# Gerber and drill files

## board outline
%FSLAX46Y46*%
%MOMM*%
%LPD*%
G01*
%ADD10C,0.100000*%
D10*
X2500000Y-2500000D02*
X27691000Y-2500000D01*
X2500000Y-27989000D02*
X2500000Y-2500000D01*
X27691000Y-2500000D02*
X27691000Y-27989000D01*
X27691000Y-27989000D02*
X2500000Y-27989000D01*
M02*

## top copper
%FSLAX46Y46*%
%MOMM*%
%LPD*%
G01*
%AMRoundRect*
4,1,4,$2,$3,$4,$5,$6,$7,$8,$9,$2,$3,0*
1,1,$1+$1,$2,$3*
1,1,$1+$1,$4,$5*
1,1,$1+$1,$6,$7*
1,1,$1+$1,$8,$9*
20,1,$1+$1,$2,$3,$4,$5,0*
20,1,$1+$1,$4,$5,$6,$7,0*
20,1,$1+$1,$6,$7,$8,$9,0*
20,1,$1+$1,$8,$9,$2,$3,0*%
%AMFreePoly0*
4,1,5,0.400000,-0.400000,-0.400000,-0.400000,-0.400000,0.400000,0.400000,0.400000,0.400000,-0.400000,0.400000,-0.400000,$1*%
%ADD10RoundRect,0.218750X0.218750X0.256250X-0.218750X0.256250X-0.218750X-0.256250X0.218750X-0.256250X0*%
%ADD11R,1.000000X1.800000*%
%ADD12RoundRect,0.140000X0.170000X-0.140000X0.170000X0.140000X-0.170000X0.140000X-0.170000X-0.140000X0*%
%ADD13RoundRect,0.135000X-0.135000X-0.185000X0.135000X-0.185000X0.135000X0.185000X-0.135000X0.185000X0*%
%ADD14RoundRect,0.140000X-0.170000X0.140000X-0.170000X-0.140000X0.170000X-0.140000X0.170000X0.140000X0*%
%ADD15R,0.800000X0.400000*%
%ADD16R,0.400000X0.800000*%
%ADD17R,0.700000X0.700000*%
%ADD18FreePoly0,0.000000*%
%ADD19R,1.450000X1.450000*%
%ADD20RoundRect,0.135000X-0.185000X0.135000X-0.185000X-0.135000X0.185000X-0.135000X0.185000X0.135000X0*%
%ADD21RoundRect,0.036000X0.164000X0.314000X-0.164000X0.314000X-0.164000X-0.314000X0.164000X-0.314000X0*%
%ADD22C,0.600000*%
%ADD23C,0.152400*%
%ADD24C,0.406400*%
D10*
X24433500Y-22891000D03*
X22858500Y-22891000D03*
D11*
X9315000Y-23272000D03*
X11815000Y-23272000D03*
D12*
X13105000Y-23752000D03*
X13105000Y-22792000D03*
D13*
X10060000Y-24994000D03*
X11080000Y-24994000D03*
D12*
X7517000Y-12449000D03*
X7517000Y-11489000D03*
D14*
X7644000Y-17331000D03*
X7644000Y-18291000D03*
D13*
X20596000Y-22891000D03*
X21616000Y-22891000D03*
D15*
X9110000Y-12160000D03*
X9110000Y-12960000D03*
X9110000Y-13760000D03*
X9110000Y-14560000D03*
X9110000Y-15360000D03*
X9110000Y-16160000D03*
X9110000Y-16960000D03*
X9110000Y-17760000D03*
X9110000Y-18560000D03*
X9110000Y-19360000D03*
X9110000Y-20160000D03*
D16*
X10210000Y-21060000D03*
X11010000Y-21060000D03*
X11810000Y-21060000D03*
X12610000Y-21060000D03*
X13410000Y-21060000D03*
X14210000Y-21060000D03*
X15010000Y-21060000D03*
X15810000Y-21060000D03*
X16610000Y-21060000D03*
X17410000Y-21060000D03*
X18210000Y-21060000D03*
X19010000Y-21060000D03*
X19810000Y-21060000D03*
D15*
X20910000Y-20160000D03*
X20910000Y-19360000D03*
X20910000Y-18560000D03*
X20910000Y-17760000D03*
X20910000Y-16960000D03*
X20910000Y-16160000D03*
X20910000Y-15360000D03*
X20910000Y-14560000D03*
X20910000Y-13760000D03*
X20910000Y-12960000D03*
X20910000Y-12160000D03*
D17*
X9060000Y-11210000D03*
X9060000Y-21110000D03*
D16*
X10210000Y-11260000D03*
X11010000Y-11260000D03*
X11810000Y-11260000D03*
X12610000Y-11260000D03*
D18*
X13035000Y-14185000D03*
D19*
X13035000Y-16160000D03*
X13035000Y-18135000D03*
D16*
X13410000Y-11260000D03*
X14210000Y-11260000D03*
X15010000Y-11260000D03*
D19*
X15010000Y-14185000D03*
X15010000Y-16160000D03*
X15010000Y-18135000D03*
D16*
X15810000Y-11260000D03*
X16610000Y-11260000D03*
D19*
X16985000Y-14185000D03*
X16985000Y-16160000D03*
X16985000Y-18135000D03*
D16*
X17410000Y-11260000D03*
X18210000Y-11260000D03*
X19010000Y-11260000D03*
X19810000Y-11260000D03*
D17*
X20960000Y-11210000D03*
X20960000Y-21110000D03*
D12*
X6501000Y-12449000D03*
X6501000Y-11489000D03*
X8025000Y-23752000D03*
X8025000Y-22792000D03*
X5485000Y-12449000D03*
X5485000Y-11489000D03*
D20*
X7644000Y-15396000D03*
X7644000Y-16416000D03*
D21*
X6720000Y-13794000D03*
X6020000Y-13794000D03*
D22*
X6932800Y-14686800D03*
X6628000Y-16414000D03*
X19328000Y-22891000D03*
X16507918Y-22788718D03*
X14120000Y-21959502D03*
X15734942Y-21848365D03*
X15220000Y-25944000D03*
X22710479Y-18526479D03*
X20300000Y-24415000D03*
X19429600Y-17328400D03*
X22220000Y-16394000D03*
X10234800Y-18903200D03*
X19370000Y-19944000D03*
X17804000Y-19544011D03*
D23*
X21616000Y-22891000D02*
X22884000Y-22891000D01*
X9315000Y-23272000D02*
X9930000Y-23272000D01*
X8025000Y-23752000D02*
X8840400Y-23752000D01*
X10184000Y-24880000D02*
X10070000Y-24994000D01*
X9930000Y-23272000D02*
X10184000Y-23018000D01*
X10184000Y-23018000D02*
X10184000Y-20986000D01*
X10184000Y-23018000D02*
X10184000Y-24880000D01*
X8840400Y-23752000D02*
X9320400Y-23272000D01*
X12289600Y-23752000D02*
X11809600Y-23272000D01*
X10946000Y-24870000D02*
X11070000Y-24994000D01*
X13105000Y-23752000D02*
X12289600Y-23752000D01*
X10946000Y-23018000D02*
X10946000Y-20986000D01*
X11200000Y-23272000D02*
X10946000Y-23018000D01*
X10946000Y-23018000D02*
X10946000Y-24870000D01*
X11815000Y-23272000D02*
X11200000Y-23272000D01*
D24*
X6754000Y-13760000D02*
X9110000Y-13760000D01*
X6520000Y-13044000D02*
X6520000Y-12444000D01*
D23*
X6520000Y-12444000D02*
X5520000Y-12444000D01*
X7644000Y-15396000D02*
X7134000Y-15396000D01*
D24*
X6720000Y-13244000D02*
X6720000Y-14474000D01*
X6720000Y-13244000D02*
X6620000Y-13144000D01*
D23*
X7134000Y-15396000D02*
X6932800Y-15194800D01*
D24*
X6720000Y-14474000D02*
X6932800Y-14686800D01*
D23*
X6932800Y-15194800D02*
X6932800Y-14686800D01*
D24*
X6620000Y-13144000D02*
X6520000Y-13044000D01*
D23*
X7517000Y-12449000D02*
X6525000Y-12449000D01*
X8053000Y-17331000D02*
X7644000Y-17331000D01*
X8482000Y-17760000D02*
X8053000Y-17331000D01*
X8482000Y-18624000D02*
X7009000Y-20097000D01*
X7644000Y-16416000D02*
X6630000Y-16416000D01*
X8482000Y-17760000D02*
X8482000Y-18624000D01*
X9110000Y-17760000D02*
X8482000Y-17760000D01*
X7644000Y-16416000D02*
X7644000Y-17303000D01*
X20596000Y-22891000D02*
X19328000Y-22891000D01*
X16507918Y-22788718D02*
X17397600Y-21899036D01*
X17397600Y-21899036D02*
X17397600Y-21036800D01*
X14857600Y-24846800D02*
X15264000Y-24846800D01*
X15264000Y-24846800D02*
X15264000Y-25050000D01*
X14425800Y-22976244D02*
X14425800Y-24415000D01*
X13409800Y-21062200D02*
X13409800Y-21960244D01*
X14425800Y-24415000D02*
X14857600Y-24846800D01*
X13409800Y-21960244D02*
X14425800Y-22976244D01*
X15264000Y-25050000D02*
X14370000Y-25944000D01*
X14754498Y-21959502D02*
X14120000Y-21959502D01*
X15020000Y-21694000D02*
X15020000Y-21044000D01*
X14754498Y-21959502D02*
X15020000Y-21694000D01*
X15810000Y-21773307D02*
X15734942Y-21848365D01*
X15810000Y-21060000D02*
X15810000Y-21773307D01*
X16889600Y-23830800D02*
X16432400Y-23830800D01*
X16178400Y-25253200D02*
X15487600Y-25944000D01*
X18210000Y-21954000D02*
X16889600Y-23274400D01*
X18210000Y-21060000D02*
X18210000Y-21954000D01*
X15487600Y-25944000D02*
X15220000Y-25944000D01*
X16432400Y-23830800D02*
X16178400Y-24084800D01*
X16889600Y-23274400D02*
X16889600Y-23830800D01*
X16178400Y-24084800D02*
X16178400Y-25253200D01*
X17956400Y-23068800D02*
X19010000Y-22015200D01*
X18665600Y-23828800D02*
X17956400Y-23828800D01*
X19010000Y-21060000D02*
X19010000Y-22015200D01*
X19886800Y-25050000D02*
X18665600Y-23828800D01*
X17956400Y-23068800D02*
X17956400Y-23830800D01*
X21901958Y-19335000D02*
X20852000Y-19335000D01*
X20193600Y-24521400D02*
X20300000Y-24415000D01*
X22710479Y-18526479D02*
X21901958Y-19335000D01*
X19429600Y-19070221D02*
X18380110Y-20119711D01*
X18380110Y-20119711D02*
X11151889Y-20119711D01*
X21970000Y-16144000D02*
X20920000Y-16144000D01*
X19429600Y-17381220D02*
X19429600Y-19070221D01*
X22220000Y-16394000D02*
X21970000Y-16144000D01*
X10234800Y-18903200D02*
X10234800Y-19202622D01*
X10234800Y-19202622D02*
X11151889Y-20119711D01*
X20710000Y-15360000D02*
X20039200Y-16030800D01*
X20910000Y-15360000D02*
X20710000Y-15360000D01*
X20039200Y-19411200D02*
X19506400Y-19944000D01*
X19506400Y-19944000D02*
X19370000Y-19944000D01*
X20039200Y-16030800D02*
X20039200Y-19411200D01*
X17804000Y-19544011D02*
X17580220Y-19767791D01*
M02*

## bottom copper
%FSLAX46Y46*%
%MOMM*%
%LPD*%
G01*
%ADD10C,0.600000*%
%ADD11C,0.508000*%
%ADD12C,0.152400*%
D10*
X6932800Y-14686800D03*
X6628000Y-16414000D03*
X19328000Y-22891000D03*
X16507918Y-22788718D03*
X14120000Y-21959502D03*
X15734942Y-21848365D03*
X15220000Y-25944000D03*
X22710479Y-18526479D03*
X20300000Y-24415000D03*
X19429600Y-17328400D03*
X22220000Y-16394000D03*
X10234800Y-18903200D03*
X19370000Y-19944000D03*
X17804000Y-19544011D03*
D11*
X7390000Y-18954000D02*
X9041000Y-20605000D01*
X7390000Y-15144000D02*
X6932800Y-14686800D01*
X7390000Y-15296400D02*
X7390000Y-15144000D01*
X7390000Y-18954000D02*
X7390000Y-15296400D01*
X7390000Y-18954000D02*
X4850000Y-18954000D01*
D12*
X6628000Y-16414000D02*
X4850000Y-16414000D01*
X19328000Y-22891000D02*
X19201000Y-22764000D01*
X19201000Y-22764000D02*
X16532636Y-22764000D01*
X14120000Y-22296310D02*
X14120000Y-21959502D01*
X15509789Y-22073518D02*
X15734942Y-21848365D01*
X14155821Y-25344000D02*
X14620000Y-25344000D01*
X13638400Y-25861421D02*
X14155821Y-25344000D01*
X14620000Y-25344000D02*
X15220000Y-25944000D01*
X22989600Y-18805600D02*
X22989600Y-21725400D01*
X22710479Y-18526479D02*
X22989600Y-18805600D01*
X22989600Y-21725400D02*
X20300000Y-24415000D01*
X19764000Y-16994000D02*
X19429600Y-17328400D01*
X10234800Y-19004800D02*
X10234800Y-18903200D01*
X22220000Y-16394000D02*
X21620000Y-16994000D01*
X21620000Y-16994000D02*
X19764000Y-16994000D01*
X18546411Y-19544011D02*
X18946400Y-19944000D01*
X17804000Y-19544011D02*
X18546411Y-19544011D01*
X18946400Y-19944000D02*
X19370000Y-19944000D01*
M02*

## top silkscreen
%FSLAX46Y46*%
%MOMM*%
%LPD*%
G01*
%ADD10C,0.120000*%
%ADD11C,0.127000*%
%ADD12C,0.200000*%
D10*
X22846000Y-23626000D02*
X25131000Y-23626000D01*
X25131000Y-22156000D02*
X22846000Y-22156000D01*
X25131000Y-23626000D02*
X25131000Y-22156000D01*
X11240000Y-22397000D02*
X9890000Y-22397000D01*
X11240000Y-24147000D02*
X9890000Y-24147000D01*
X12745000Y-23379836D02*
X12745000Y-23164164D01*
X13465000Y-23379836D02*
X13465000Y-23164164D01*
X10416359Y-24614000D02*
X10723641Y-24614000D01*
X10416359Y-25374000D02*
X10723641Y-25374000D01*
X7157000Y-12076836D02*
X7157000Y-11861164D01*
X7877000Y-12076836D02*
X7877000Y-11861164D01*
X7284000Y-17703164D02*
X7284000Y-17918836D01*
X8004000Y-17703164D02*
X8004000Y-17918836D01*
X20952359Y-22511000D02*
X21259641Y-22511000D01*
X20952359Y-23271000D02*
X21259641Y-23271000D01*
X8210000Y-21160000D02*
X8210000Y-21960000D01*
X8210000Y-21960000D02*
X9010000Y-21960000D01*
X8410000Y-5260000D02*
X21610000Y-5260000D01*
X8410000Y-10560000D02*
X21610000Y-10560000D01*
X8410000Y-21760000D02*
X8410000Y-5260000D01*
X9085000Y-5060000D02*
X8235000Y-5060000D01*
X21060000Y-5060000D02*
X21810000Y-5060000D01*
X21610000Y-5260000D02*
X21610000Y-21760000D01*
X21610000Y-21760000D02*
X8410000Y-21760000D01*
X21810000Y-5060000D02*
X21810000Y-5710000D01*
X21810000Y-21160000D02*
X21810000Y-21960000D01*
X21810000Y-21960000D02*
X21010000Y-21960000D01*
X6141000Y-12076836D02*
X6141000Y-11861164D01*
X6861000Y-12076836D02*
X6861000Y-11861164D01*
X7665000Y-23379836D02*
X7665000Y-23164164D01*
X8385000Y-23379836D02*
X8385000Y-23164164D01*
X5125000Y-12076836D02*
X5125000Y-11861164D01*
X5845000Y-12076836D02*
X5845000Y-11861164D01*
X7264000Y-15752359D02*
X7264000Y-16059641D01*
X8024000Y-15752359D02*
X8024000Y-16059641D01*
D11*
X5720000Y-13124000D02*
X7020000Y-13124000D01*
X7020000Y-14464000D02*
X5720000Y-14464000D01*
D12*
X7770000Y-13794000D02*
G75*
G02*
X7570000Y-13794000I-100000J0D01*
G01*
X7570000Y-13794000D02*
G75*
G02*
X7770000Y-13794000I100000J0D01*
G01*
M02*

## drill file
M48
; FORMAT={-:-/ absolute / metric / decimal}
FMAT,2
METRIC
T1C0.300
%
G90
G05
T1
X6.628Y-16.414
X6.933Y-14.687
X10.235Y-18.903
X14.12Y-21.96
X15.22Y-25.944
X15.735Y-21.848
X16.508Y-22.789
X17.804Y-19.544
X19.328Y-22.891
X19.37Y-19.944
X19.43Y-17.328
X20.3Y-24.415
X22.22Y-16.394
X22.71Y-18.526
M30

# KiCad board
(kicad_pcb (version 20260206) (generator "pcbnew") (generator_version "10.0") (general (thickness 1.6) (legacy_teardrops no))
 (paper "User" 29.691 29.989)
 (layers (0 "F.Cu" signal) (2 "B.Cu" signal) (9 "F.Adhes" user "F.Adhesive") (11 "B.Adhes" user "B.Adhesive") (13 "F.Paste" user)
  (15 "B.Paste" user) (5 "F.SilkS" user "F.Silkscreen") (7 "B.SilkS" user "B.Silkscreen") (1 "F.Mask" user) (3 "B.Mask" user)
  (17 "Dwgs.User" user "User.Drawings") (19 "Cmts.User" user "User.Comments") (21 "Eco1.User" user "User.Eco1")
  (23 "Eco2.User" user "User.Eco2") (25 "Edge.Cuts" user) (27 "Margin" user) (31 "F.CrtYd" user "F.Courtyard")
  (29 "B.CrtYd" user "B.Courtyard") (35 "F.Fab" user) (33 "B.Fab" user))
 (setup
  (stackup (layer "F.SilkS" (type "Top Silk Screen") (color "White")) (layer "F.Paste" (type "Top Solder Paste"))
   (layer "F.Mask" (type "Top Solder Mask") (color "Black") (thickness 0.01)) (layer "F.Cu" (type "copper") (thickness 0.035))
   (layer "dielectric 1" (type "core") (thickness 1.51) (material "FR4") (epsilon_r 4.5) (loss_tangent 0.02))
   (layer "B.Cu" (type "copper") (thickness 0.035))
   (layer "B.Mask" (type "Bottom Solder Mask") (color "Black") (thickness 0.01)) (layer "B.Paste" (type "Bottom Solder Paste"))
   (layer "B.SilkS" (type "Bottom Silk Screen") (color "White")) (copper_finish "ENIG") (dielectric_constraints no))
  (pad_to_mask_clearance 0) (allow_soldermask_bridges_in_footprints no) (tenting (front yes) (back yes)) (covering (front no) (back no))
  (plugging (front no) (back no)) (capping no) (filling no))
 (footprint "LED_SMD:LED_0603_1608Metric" (layer "F.Cu") (at 23.646 22.891 180)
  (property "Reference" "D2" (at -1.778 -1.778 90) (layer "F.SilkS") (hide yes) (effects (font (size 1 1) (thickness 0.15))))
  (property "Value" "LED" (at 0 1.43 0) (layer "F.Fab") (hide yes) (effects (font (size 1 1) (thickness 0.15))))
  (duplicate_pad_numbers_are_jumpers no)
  (fp_line (start 0.8 -0.735) (end -1.485 -0.735) (stroke (width 0.12) (type solid)) (layer "F.SilkS"))
  (fp_line (start -1.485 0.735) (end 0.8 0.735) (stroke (width 0.12) (type solid)) (layer "F.SilkS"))
  (fp_line (start -1.485 -0.735) (end -1.485 0.735) (stroke (width 0.12) (type solid)) (layer "F.SilkS"))
  (pad "1" smd roundrect (at -0.7875 0 180) (size 0.875 0.95) (layers "F.Cu" "F.Mask" "F.Paste") (roundrect_rratio 0.25) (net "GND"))
  (pad "2" smd roundrect (at 0.7875 0 180) (size 0.875 0.95) (layers "F.Cu" "F.Mask" "F.Paste") (roundrect_rratio 0.25)
   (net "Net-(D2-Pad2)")))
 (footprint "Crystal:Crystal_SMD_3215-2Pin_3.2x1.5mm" (layer "F.Cu") (at 10.565 23.272 180)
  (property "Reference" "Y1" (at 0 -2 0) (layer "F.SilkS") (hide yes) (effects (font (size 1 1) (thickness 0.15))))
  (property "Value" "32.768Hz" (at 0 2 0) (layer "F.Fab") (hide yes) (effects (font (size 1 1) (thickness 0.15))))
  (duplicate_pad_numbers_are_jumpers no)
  (fp_line (start -0.675 0.875) (end 0.675 0.875) (stroke (width 0.12) (type solid)) (layer "F.SilkS"))
  (fp_line (start -0.675 -0.875) (end 0.675 -0.875) (stroke (width 0.12) (type solid)) (layer "F.SilkS"))
  (pad "1" smd rect (at 1.25 0 180) (size 1 1.8) (layers "F.Cu" "F.Mask" "F.Paste") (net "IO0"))
  (pad "2" smd rect (at -1.25 0 180) (size 1 1.8) (layers "F.Cu" "F.Mask" "F.Paste") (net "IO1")))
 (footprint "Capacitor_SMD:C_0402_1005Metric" (layer "F.Cu") (at 13.105 23.272 90)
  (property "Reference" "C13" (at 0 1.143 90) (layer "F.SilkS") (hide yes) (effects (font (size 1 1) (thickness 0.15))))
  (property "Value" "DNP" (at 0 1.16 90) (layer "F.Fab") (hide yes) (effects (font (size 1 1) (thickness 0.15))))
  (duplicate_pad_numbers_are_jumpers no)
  (fp_line (start -0.107836 -0.36) (end 0.107836 -0.36) (stroke (width 0.12) (type solid)) (layer "F.SilkS"))
  (fp_line (start -0.107836 0.36) (end 0.107836 0.36) (stroke (width 0.12) (type solid)) (layer "F.SilkS"))
  (pad "1" smd roundrect (at -0.48 0 90) (size 0.56 0.62) (layers "F.Cu" "F.Mask" "F.Paste") (roundrect_rratio 0.25) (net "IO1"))
  (pad "2" smd roundrect (at 0.48 0 90) (size 0.56 0.62) (layers "F.Cu" "F.Mask" "F.Paste") (roundrect_rratio 0.25) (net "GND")))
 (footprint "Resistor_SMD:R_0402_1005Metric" (layer "F.Cu") (at 10.57 24.994)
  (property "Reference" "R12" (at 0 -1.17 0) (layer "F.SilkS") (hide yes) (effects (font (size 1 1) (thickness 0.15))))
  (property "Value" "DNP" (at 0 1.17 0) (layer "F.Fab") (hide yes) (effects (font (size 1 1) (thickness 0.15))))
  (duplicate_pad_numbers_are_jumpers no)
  (fp_line (start -0.153641 -0.38) (end 0.153641 -0.38) (stroke (width 0.12) (type solid)) (layer "F.SilkS"))
  (fp_line (start -0.153641 0.38) (end 0.153641 0.38) (stroke (width 0.12) (type solid)) (layer "F.SilkS"))
  (pad "1" smd roundrect (at -0.51 0) (size 0.54 0.64) (layers "F.Cu" "F.Mask" "F.Paste") (roundrect_rratio 0.25) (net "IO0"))
  (pad "2" smd roundrect (at 0.51 0) (size 0.54 0.64) (layers "F.Cu" "F.Mask" "F.Paste") (roundrect_rratio 0.25) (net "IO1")))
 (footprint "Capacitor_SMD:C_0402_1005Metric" (layer "F.Cu") (at 7.517 11.969 90)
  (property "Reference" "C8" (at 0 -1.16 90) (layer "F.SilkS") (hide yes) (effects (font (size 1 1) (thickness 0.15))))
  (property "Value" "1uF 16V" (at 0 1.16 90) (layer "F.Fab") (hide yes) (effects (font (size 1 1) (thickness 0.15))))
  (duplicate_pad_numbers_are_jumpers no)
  (fp_line (start -0.107836 -0.36) (end 0.107836 -0.36) (stroke (width 0.12) (type solid)) (layer "F.SilkS"))
  (fp_line (start -0.107836 0.36) (end 0.107836 0.36) (stroke (width 0.12) (type solid)) (layer "F.SilkS"))
  (pad "1" smd roundrect (at -0.48 0 90) (size 0.56 0.62) (layers "F.Cu" "F.Mask" "F.Paste") (roundrect_rratio 0.25) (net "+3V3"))
  (pad "2" smd roundrect (at 0.48 0 90) (size 0.56 0.62) (layers "F.Cu" "F.Mask" "F.Paste") (roundrect_rratio 0.25) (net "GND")))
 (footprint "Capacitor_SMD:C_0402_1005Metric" (layer "F.Cu") (at 7.644 17.811 -90)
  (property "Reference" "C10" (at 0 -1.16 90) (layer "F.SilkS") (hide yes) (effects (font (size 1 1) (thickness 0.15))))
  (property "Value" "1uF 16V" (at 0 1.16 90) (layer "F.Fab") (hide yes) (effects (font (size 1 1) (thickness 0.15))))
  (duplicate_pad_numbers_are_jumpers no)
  (fp_line (start -0.107836 0.36) (end 0.107836 0.36) (stroke (width 0.12) (type solid)) (layer "F.SilkS"))
  (fp_line (start -0.107836 -0.36) (end 0.107836 -0.36) (stroke (width 0.12) (type solid)) (layer "F.SilkS"))
  (pad "1" smd roundrect (at -0.48 0 270) (size 0.56 0.62) (layers "F.Cu" "F.Mask" "F.Paste") (roundrect_rratio 0.25) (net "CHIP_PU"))
  (pad "2" smd roundrect (at 0.48 0 270) (size 0.56 0.62) (layers "F.Cu" "F.Mask" "F.Paste") (roundrect_rratio 0.25) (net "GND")))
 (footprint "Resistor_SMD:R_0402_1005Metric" (layer "F.Cu") (at 21.106 22.891)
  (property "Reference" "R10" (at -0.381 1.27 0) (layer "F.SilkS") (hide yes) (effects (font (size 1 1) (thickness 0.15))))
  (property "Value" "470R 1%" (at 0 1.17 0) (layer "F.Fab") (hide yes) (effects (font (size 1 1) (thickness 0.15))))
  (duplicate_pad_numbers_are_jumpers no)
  (fp_line (start -0.153641 -0.38) (end 0.153641 -0.38) (stroke (width 0.12) (type solid)) (layer "F.SilkS"))
  (fp_line (start -0.153641 0.38) (end 0.153641 0.38) (stroke (width 0.12) (type solid)) (layer "F.SilkS"))
  (pad "1" smd roundrect (at -0.51 0) (size 0.54 0.64) (layers "F.Cu" "F.Mask" "F.Paste") (roundrect_rratio 0.25) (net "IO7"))
  (pad "2" smd roundrect (at 0.51 0) (size 0.54 0.64) (layers "F.Cu" "F.Mask" "F.Paste") (roundrect_rratio 0.25) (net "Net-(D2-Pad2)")))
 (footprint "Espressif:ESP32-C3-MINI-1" (layer "F.Cu") (at 15.01 16.16)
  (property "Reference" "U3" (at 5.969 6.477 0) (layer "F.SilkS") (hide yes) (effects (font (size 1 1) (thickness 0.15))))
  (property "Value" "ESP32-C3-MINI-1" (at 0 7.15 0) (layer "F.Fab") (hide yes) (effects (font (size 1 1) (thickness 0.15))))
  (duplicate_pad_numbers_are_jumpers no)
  (fp_line (start -6.8 5) (end -6.8 5.8) (stroke (width 0.12) (type solid)) (layer "F.SilkS"))
  (fp_line (start -6.8 5.8) (end -6 5.8) (stroke (width 0.12) (type solid)) (layer "F.SilkS"))
  (fp_line (start -6.6 -10.9) (end 6.6 -10.9) (stroke (width 0.12) (type solid)) (layer "F.SilkS"))
  (fp_line (start -6.6 -5.6) (end 6.6 -5.6) (stroke (width 0.12) (type solid)) (layer "F.SilkS"))
  (fp_line (start -6.6 5.6) (end -6.6 -10.9) (stroke (width 0.12) (type solid)) (layer "F.SilkS"))
  (fp_line (start -5.925 -11.1) (end -6.775 -11.1) (stroke (width 0.12) (type solid)) (layer "F.SilkS"))
  (fp_line (start 6.05 -11.1) (end 6.8 -11.1) (stroke (width 0.12) (type solid)) (layer "F.SilkS"))
  (fp_line (start 6.6 -10.9) (end 6.6 5.6) (stroke (width 0.12) (type solid)) (layer "F.SilkS"))
  (fp_line (start 6.6 5.6) (end -6.6 5.6) (stroke (width 0.12) (type solid)) (layer "F.SilkS"))
  (fp_line (start 6.8 -11.1) (end 6.8 -10.45) (stroke (width 0.12) (type solid)) (layer "F.SilkS"))
  (fp_line (start 6.8 5) (end 6.8 5.8) (stroke (width 0.12) (type solid)) (layer "F.SilkS"))
  (fp_line (start 6.8 5.8) (end 6 5.8) (stroke (width 0.12) (type solid)) (layer "F.SilkS"))
  (pad "1" smd rect (at -5.9 -4 90) (size 0.4 0.8) (layers "F.Cu" "F.Mask" "F.Paste") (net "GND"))
  (pad "2" smd rect (at -5.9 -3.2 90) (size 0.4 0.8) (layers "F.Cu" "F.Mask" "F.Paste") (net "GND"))
  (pad "3" smd rect (at -5.9 -2.4 90) (size 0.4 0.8) (layers "F.Cu" "F.Mask" "F.Paste") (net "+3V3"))
  (pad "4" smd rect (at -5.9 -1.6 90) (size 0.4 0.8) (layers "F.Cu" "F.Mask" "F.Paste") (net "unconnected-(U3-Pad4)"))
  (pad "5" smd rect (at -5.9 -0.8 90) (size 0.4 0.8) (layers "F.Cu" "F.Mask" "F.Paste") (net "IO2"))
  (pad "6" smd rect (at -5.9 0 90) (size 0.4 0.8) (layers "F.Cu" "F.Mask" "F.Paste") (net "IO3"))
  (pad "7" smd rect (at -5.9 0.8 90) (size 0.4 0.8) (layers "F.Cu" "F.Mask" "F.Paste") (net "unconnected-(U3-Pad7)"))
  (pad "8" smd rect (at -5.9 1.6 90) (size 0.4 0.8) (layers "F.Cu" "F.Mask" "F.Paste") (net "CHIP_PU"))
  (pad "9" smd rect (at -5.9 2.4 90) (size 0.4 0.8) (layers "F.Cu" "F.Mask" "F.Paste") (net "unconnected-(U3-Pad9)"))
  (pad "10" smd rect (at -5.9 3.2 90) (size 0.4 0.8) (layers "F.Cu" "F.Mask" "F.Paste") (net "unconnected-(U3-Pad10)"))
  (pad "11" smd rect (at -5.9 4 90) (size 0.4 0.8) (layers "F.Cu" "F.Mask" "F.Paste") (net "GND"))
  (pad "12" smd rect (at -4.8 4.9) (size 0.4 0.8) (layers "F.Cu" "F.Mask" "F.Paste") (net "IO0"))
  (pad "13" smd rect (at -4 4.9) (size 0.4 0.8) (layers "F.Cu" "F.Mask" "F.Paste") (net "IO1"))
  (pad "14" smd rect (at -3.2 4.9) (size 0.4 0.8) (layers "F.Cu" "F.Mask" "F.Paste") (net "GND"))
  (pad "15" smd rect (at -2.4 4.9) (size 0.4 0.8) (layers "F.Cu" "F.Mask" "F.Paste") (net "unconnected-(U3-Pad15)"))
  (pad "16" smd rect (at -1.6 4.9) (size 0.4 0.8) (layers "F.Cu" "F.Mask" "F.Paste") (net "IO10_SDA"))
  (pad "17" smd rect (at -0.8 4.9) (size 0.4 0.8) (layers "F.Cu" "F.Mask" "F.Paste") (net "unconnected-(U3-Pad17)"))
  (pad "18" smd rect (at 0 4.9) (size 0.4 0.8) (layers "F.Cu" "F.Mask" "F.Paste") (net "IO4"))
  (pad "19" smd rect (at 0.8 4.9) (size 0.4 0.8) (layers "F.Cu" "F.Mask" "F.Paste") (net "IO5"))
  (pad "20" smd rect (at 1.6 4.9) (size 0.4 0.8) (layers "F.Cu" "F.Mask" "F.Paste") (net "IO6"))
  (pad "21" smd rect (at 2.4 4.9) (size 0.4 0.8) (layers "F.Cu" "F.Mask" "F.Paste") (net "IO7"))
  (pad "22" smd rect (at 3.2 4.9) (size 0.4 0.8) (layers "F.Cu" "F.Mask" "F.Paste") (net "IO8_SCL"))
  (pad "23" smd rect (at 4 4.9) (size 0.4 0.8) (layers "F.Cu" "F.Mask" "F.Paste") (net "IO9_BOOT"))
  (pad "24" smd rect (at 4.8 4.9) (size 0.4 0.8) (layers "F.Cu" "F.Mask" "F.Paste") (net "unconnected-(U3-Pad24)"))
  (pad "25" smd rect (at 5.9 4 90) (size 0.4 0.8) (layers "F.Cu" "F.Mask" "F.Paste") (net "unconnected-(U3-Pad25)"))
  (pad "26" smd rect (at 5.9 3.2 90) (size 0.4 0.8) (layers "F.Cu" "F.Mask" "F.Paste") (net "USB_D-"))
  (pad "27" smd rect (at 5.9 2.4 90) (size 0.4 0.8) (layers "F.Cu" "F.Mask" "F.Paste") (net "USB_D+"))
  (pad "28" smd rect (at 5.9 1.6 90) (size 0.4 0.8) (layers "F.Cu" "F.Mask" "F.Paste") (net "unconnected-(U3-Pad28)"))
  (pad "29" smd rect (at 5.9 0.8 90) (size 0.4 0.8) (layers "F.Cu" "F.Mask" "F.Paste") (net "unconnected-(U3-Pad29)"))
  (pad "30" smd rect (at 5.9 0 90) (size 0.4 0.8) (layers "F.Cu" "F.Mask" "F.Paste") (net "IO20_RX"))
  (pad "31" smd rect (at 5.9 -0.8 90) (size 0.4 0.8) (layers "F.Cu" "F.Mask" "F.Paste") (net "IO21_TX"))
  (pad "32" smd rect (at 5.9 -1.6 90) (size 0.4 0.8) (layers "F.Cu" "F.Mask" "F.Paste") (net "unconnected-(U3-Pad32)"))
  (pad "33" smd rect (at 5.9 -2.4 90) (size 0.4 0.8) (layers "F.Cu" "F.Mask" "F.Paste") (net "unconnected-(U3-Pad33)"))
  (pad "34" smd rect (at 5.9 -3.2 90) (size 0.4 0.8) (layers "F.Cu" "F.Mask" "F.Paste") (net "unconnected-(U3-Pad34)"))
  (pad "35" smd rect (at 5.9 -4 90) (size 0.4 0.8) (layers "F.Cu" "F.Mask" "F.Paste") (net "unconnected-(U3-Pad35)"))
  (pad "36" smd rect (at -5.95 -4.95 90) (size 0.7 0.7) (layers "F.Cu" "F.Mask" "F.Paste") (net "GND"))
  (pad "36" smd rect (at -5.95 4.95 90) (size 0.7 0.7) (layers "F.Cu" "F.Mask" "F.Paste") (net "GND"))
  (pad "36" smd rect (at -4.8 -4.9) (size 0.4 0.8) (layers "F.Cu" "F.Mask" "F.Paste") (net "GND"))
  (pad "36" smd rect (at -4 -4.9) (size 0.4 0.8) (layers "F.Cu" "F.Mask" "F.Paste") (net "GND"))
  (pad "36" smd rect (at -3.2 -4.9) (size 0.4 0.8) (layers "F.Cu" "F.Mask" "F.Paste") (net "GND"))
  (pad "36" smd rect (at -2.4 -4.9) (size 0.4 0.8) (layers "F.Cu" "F.Mask" "F.Paste") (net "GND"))
  (pad "36" smd custom (at -1.975 -1.975) (size 0.8 0.8) (layers "F.Cu" "F.Mask" "F.Paste") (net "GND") (zone_connect 2)
   (options (clearance outline) (anchor rect)) (primitives))
  (pad "36" smd rect (at -1.975 0 90) (size 1.45 1.45) (layers "F.Cu" "F.Mask" "F.Paste") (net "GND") (zone_connect 2))
  (pad "36" smd rect (at -1.975 1.975 90) (size 1.45 1.45) (layers "F.Cu" "F.Mask" "F.Paste") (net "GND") (zone_connect 2))
  (pad "36" smd rect (at -1.6 -4.9) (size 0.4 0.8) (layers "F.Cu" "F.Mask" "F.Paste") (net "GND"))
  (pad "36" smd rect (at -0.8 -4.9) (size 0.4 0.8) (layers "F.Cu" "F.Mask" "F.Paste") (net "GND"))
  (pad "36" smd rect (at 0 -4.9) (size 0.4 0.8) (layers "F.Cu" "F.Mask" "F.Paste") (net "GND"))
  (pad "36" smd rect (at 0 -1.975 90) (size 1.45 1.45) (layers "F.Cu" "F.Mask" "F.Paste") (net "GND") (zone_connect 2))
  (pad "36" smd rect (at 0 0 90) (size 1.45 1.45) (layers "F.Cu" "F.Mask" "F.Paste") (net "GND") (zone_connect 2))
  (pad "36" smd rect (at 0 1.975 90) (size 1.45 1.45) (layers "F.Cu" "F.Mask" "F.Paste") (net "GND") (zone_connect 2))
  (pad "36" smd rect (at 0.8 -4.9) (size 0.4 0.8) (layers "F.Cu" "F.Mask" "F.Paste") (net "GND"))
  (pad "36" smd rect (at 1.6 -4.9) (size 0.4 0.8) (layers "F.Cu" "F.Mask" "F.Paste") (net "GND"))
  (pad "36" smd rect (at 1.975 -1.975 90) (size 1.45 1.45) (layers "F.Cu" "F.Mask" "F.Paste") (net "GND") (zone_connect 2))
  (pad "36" smd rect (at 1.975 0 90) (size 1.45 1.45) (layers "F.Cu" "F.Mask" "F.Paste") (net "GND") (zone_connect 2))
  (pad "36" smd rect (at 1.975 1.975 90) (size 1.45 1.45) (layers "F.Cu" "F.Mask" "F.Paste") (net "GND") (zone_connect 2))
  (pad "36" smd rect (at 2.4 -4.9) (size 0.4 0.8) (layers "F.Cu" "F.Mask" "F.Paste") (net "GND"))
  (pad "36" smd rect (at 3.2 -4.9) (size 0.4 0.8) (layers "F.Cu" "F.Mask" "F.Paste") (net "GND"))
  (pad "36" smd rect (at 4 -4.9) (size 0.4 0.8) (layers "F.Cu" "F.Mask" "F.Paste") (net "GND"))
  (pad "36" smd rect (at 4.8 -4.9) (size 0.4 0.8) (layers "F.Cu" "F.Mask" "F.Paste") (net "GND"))
  (pad "36" smd rect (at 5.95 -4.95 90) (size 0.7 0.7) (layers "F.Cu" "F.Mask" "F.Paste") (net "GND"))
  (pad "36" smd rect (at 5.95 4.95 90) (size 0.7 0.7) (layers "F.Cu" "F.Mask" "F.Paste") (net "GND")))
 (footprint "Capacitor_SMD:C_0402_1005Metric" (layer "F.Cu") (at 6.501 11.969 90)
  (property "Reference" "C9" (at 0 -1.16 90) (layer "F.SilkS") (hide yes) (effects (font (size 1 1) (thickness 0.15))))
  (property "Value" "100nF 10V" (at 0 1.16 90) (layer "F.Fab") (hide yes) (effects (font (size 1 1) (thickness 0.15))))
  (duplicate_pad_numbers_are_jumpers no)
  (fp_line (start -0.107836 -0.36) (end 0.107836 -0.36) (stroke (width 0.12) (type solid)) (layer "F.SilkS"))
  (fp_line (start -0.107836 0.36) (end 0.107836 0.36) (stroke (width 0.12) (type solid)) (layer "F.SilkS"))
  (pad "1" smd roundrect (at -0.48 0 90) (size 0.56 0.62) (layers "F.Cu" "F.Mask" "F.Paste") (roundrect_rratio 0.25) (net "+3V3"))
  (pad "2" smd roundrect (at 0.48 0 90) (size 0.56 0.62) (layers "F.Cu" "F.Mask" "F.Paste") (roundrect_rratio 0.25) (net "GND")))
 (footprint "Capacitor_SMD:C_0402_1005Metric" (layer "F.Cu") (at 8.025 23.272 90)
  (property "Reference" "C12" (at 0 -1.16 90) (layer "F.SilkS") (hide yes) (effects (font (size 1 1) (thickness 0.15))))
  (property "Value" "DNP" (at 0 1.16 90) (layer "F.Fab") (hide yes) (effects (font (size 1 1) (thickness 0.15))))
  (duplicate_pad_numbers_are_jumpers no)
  (fp_line (start -0.107836 -0.36) (end 0.107836 -0.36) (stroke (width 0.12) (type solid)) (layer "F.SilkS"))
  (fp_line (start -0.107836 0.36) (end 0.107836 0.36) (stroke (width 0.12) (type solid)) (layer "F.SilkS"))
  (pad "1" smd roundrect (at -0.48 0 90) (size 0.56 0.62) (layers "F.Cu" "F.Mask" "F.Paste") (roundrect_rratio 0.25) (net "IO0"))
  (pad "2" smd roundrect (at 0.48 0 90) (size 0.56 0.62) (layers "F.Cu" "F.Mask" "F.Paste") (roundrect_rratio 0.25) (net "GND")))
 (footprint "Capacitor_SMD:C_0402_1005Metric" (layer "F.Cu") (at 5.485 11.969 90)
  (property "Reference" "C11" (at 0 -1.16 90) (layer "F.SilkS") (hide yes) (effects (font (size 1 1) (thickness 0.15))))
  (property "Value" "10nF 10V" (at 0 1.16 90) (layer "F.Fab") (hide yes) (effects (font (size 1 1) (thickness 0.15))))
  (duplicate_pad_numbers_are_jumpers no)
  (fp_line (start -0.107836 -0.36) (end 0.107836 -0.36) (stroke (width 0.12) (type solid)) (layer "F.SilkS"))
  (fp_line (start -0.107836 0.36) (end 0.107836 0.36) (stroke (width 0.12) (type solid)) (layer "F.SilkS"))
  (pad "1" smd roundrect (at -0.48 0 90) (size 0.56 0.62) (layers "F.Cu" "F.Mask" "F.Paste") (roundrect_rratio 0.25) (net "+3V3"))
  (pad "2" smd roundrect (at 0.48 0 90) (size 0.56 0.62) (layers "F.Cu" "F.Mask" "F.Paste") (roundrect_rratio 0.25) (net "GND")))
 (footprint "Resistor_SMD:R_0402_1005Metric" (layer "F.Cu") (at 7.644 15.906 -90)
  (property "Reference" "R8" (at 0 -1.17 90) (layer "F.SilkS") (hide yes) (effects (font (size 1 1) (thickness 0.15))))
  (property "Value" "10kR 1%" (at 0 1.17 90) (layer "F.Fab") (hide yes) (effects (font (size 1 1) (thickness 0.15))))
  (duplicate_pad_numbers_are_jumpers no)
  (fp_line (start -0.153641 0.38) (end 0.153641 0.38) (stroke (width 0.12) (type solid)) (layer "F.SilkS"))
  (fp_line (start -0.153641 -0.38) (end 0.153641 -0.38) (stroke (width 0.12) (type solid)) (layer "F.SilkS"))
  (pad "1" smd roundrect (at -0.51 0 270) (size 0.54 0.64) (layers "F.Cu" "F.Mask" "F.Paste") (roundrect_rratio 0.25) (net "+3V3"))
  (pad "2" smd roundrect (at 0.51 0 270) (size 0.54 0.64) (layers "F.Cu" "F.Mask" "F.Paste") (roundrect_rratio 0.25) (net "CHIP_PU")))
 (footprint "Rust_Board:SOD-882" (layer "F.Cu") (at 6.37 13.794 180)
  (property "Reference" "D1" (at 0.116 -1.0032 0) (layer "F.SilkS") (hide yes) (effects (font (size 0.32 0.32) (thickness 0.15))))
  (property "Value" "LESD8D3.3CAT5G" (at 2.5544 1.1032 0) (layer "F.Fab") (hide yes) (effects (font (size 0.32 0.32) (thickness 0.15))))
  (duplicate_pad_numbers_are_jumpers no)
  (fp_line (start 0.65 0.67) (end -0.65 0.67) (stroke (width 0.127) (type solid)) (layer "F.SilkS"))
  (fp_line (start -0.65 -0.67) (end 0.65 -0.67) (stroke (width 0.127) (type solid)) (layer "F.SilkS"))
  (fp_circle (center -1.3 0) (end -1.2 0) (stroke (width 0.2) (type solid)) (fill no) (layer "F.SilkS"))
  (pad "1" smd roundrect (at -0.35 0 180) (size 0.4 0.7) (layers "F.Cu") (roundrect_rratio 0.09) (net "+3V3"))
  (pad "2" smd roundrect (at 0.35 0 180) (size 0.4 0.7) (layers "F.Cu") (roundrect_rratio 0.09) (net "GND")))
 (gr_line (start 2.5 2.5) (end 27.691 2.5) (stroke (width 0.1) (type default)) (layer "Edge.Cuts"))
 (gr_line (start 2.5 27.989) (end 2.5 2.5) (stroke (width 0.1) (type default)) (layer "Edge.Cuts"))
 (gr_line (start 27.691 2.5) (end 27.691 27.989) (stroke (width 0.1) (type default)) (layer "Edge.Cuts"))
 (gr_line (start 27.691 27.989) (end 2.5 27.989) (stroke (width 0.1) (type default)) (layer "Edge.Cuts"))
 (segment (start 21.616 22.891) (end 22.884 22.891) (width 0.1524) (layer "F.Cu") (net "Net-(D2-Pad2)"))
 (segment (start 9.315 23.272) (end 9.93 23.272) (width 0.1524) (layer "F.Cu") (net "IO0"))
 (segment (start 8.025 23.752) (end 8.8404 23.752) (width 0.1524) (layer "F.Cu") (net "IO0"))
 (segment (start 10.184 24.88) (end 10.07 24.994) (width 0.1524) (layer "F.Cu") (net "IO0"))
 (segment (start 9.93 23.272) (end 10.184 23.018) (width 0.1524) (layer "F.Cu") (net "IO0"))
 (segment (start 10.184 23.018) (end 10.184 20.986) (width 0.1524) (layer "F.Cu") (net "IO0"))
 (segment (start 10.184 23.018) (end 10.184 24.88) (width 0.1524) (layer "F.Cu") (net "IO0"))
 (segment (start 8.8404 23.752) (end 9.3204 23.272) (width 0.1524) (layer "F.Cu") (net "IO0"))
 (segment (start 12.2896 23.752) (end 11.8096 23.272) (width 0.1524) (layer "F.Cu") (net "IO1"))
 (segment (start 10.946 24.87) (end 11.07 24.994) (width 0.1524) (layer "F.Cu") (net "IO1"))
 (segment (start 13.105 23.752) (end 12.2896 23.752) (width 0.1524) (layer "F.Cu") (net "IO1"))
 (segment (start 10.946 23.018) (end 10.946 20.986) (width 0.1524) (layer "F.Cu") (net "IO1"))
 (segment (start 11.2 23.272) (end 10.946 23.018) (width 0.1524) (layer "F.Cu") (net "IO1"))
 (segment (start 10.946 23.018) (end 10.946 24.87) (width 0.1524) (layer "F.Cu") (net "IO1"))
 (segment (start 11.815 23.272) (end 11.2 23.272) (width 0.1524) (layer "F.Cu") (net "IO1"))
 (segment (start 6.754 13.76) (end 9.11 13.76) (width 0.4064) (layer "F.Cu") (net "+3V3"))
 (segment (start 6.52 13.044) (end 6.52 12.444) (width 0.4064) (layer "F.Cu") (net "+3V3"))
 (segment (start 6.52 12.444) (end 5.52 12.444) (width 0.1524) (layer "F.Cu") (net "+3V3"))
 (segment (start 7.644 15.396) (end 7.134 15.396) (width 0.1524) (layer "F.Cu") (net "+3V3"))
 (segment (start 6.72 13.244) (end 6.72 14.474) (width 0.4064) (layer "F.Cu") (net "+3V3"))
 (segment (start 6.72 13.244) (end 6.62 13.144) (width 0.4064) (layer "F.Cu") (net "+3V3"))
 (segment (start 7.134 15.396) (end 6.9328 15.1948) (width 0.1524) (layer "F.Cu") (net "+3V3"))
 (segment (start 6.72 14.474) (end 6.9328 14.6868) (width 0.4064) (layer "F.Cu") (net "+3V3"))
 (segment (start 6.9328 15.1948) (end 6.9328 14.6868) (width 0.1524) (layer "F.Cu") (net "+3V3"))
 (segment (start 6.62 13.144) (end 6.52 13.044) (width 0.4064) (layer "F.Cu") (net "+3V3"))
 (segment (start 7.517 12.449) (end 6.525 12.449) (width 0.1524) (layer "F.Cu") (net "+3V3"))
 (via (at 6.9328 14.6868) (size 0.6) (drill 0.3) (layers "F.Cu" "B.Cu") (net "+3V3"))
 (segment (start 7.39 18.954) (end 9.041 20.605) (width 0.508) (layer "B.Cu") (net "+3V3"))
 (segment (start 7.39 15.144) (end 6.9328 14.6868) (width 0.508) (layer "B.Cu") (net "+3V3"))
 (segment (start 7.39 15.2964) (end 7.39 15.144) (width 0.508) (layer "B.Cu") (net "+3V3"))
 (segment (start 7.39 18.954) (end 7.39 15.2964) (width 0.508) (layer "B.Cu") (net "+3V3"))
 (segment (start 7.39 18.954) (end 4.85 18.954) (width 0.508) (layer "B.Cu") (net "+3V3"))
 (segment (start 8.053 17.331) (end 7.644 17.331) (width 0.1524) (layer "F.Cu") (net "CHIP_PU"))
 (segment (start 8.482 17.76) (end 8.053 17.331) (width 0.1524) (layer "F.Cu") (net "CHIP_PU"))
 (segment (start 8.482 18.624) (end 7.009 20.097) (width 0.1524) (layer "F.Cu") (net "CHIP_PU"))
 (segment (start 7.644 16.416) (end 6.63 16.416) (width 0.1524) (layer "F.Cu") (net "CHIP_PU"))
 (segment (start 8.482 17.76) (end 8.482 18.624) (width 0.1524) (layer "F.Cu") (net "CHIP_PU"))
 (segment (start 9.11 17.76) (end 8.482 17.76) (width 0.1524) (layer "F.Cu") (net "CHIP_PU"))
 (segment (start 7.644 16.416) (end 7.644 17.303) (width 0.1524) (layer "F.Cu") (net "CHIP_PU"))
 (via (at 6.628 16.414) (size 0.6) (drill 0.3) (layers "F.Cu" "B.Cu") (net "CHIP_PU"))
 (segment (start 6.628 16.414) (end 4.85 16.414) (width 0.1524) (layer "B.Cu") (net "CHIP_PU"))
 (segment (start 20.596 22.891) (end 19.328 22.891) (width 0.1524) (layer "F.Cu") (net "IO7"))
 (segment (start 16.507918 22.788718) (end 17.3976 21.899036) (width 0.1524) (layer "F.Cu") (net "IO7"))
 (segment (start 17.3976 21.899036) (end 17.3976 21.0368) (width 0.1524) (layer "F.Cu") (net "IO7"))
 (via (at 19.328 22.891) (size 0.6) (drill 0.3) (layers "F.Cu" "B.Cu") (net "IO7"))
 (via (at 16.507918 22.788718) (size 0.6) (drill 0.3) (layers "F.Cu" "B.Cu") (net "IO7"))
 (segment (start 19.328 22.891) (end 19.201 22.764) (width 0.1524) (layer "B.Cu") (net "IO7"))
 (segment (start 19.201 22.764) (end 16.532636 22.764) (width 0.1524) (layer "B.Cu") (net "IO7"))
 (segment (start 14.8576 24.8468) (end 15.264 24.8468) (width 0.1524) (layer "F.Cu") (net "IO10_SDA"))
 (segment (start 15.264 24.8468) (end 15.264 25.05) (width 0.1524) (layer "F.Cu") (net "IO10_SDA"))
 (segment (start 14.4258 22.976244) (end 14.4258 24.415) (width 0.1524) (layer "F.Cu") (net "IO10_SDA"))
 (segment (start 13.4098 21.0622) (end 13.4098 21.960244) (width 0.1524) (layer "F.Cu") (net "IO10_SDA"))
 (segment (start 14.4258 24.415) (end 14.8576 24.8468) (width 0.1524) (layer "F.Cu") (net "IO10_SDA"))
 (segment (start 13.4098 21.960244) (end 14.4258 22.976244) (width 0.1524) (layer "F.Cu") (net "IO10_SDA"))
 (segment (start 15.264 25.05) (end 14.37 25.944) (width 0.1524) (layer "F.Cu") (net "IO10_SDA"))
 (segment (start 14.754498 21.959502) (end 14.12 21.959502) (width 0.1524) (layer "F.Cu") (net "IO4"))
 (segment (start 15.02 21.694) (end 15.02 21.044) (width 0.1524) (layer "F.Cu") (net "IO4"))
 (segment (start 14.754498 21.959502) (end 15.02 21.694) (width 0.1524) (layer "F.Cu") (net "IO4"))
 (via (at 14.12 21.959502) (size 0.6) (drill 0.3) (layers "F.Cu" "B.Cu") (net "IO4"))
 (segment (start 14.12 22.29631) (end 14.12 21.959502) (width 0.1524) (layer "B.Cu") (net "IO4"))
 (segment (start 15.81 21.773307) (end 15.734942 21.848365) (width 0.1524) (layer "F.Cu") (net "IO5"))
 (segment (start 15.81 21.06) (end 15.81 21.773307) (width 0.1524) (layer "F.Cu") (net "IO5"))
 (via (at 15.734942 21.848365) (size 0.6) (drill 0.3) (layers "F.Cu" "B.Cu") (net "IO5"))
 (segment (start 15.509789 22.073518) (end 15.734942 21.848365) (width 0.1524) (layer "B.Cu") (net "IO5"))
 (segment (start 16.8896 23.8308) (end 16.4324 23.8308) (width 0.1524) (layer "F.Cu") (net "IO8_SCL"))
 (segment (start 16.1784 25.2532) (end 15.4876 25.944) (width 0.1524) (layer "F.Cu") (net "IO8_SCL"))
 (segment (start 18.21 21.954) (end 16.8896 23.2744) (width 0.1524) (layer "F.Cu") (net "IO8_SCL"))
 (segment (start 18.21 21.06) (end 18.21 21.954) (width 0.1524) (layer "F.Cu") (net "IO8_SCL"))
 (segment (start 15.4876 25.944) (end 15.22 25.944) (width 0.1524) (layer "F.Cu") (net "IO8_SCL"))
 (segment (start 16.4324 23.8308) (end 16.1784 24.0848) (width 0.1524) (layer "F.Cu") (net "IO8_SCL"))
 (segment (start 16.8896 23.2744) (end 16.8896 23.8308) (width 0.1524) (layer "F.Cu") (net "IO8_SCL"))
 (segment (start 16.1784 24.0848) (end 16.1784 25.2532) (width 0.1524) (layer "F.Cu") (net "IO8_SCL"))
 (via (at 15.22 25.944) (size 0.6) (drill 0.3) (layers "F.Cu" "B.Cu") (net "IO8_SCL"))
 (segment (start 14.155821 25.344) (end 14.62 25.344) (width 0.1524) (layer "B.Cu") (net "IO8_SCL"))
 (segment (start 13.6384 25.861421) (end 14.155821 25.344) (width 0.1524) (layer "B.Cu") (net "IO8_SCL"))
 (segment (start 14.62 25.344) (end 15.22 25.944) (width 0.1524) (layer "B.Cu") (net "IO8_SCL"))
 (segment (start 17.9564 23.0688) (end 19.01 22.0152) (width 0.1524) (layer "F.Cu") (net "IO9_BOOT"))
 (segment (start 18.6656 23.8288) (end 17.9564 23.8288) (width 0.1524) (layer "F.Cu") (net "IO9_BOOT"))
 (segment (start 19.01 21.06) (end 19.01 22.0152) (width 0.1524) (layer "F.Cu") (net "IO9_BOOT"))
 (segment (start 19.8868 25.05) (end 18.6656 23.8288) (width 0.1524) (layer "F.Cu") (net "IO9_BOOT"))
 (segment (start 17.9564 23.0688) (end 17.9564 23.8308) (width 0.1524) (layer "F.Cu") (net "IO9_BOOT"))
 (segment (start 21.901958 19.335) (end 20.852 19.335) (width 0.1524) (layer "F.Cu") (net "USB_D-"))
 (segment (start 20.1936 24.5214) (end 20.3 24.415) (width 0.1524) (layer "F.Cu") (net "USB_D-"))
 (segment (start 22.710479 18.526479) (end 21.901958 19.335) (width 0.1524) (layer "F.Cu") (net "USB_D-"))
 (via (at 22.710479 18.526479) (size 0.6) (drill 0.3) (layers "F.Cu" "B.Cu") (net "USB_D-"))
 (via (at 20.3 24.415) (size 0.6) (drill 0.3) (layers "F.Cu" "B.Cu") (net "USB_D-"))
 (segment (start 22.9896 18.8056) (end 22.9896 21.7254) (width 0.1524) (layer "B.Cu") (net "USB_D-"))
 (segment (start 22.710479 18.526479) (end 22.9896 18.8056) (width 0.1524) (layer "B.Cu") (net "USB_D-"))
 (segment (start 22.9896 21.7254) (end 20.3 24.415) (width 0.1524) (layer "B.Cu") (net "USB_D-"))
 (segment (start 19.4296 19.070221) (end 18.38011 20.119711) (width 0.1524) (layer "F.Cu") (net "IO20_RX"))
 (segment (start 18.38011 20.119711) (end 11.151889 20.119711) (width 0.1524) (layer "F.Cu") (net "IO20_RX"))
 (segment (start 21.97 16.144) (end 20.92 16.144) (width 0.1524) (layer "F.Cu") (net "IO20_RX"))
 (segment (start 19.4296 17.38122) (end 19.4296 19.070221) (width 0.1524) (layer "F.Cu") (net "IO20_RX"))
 (segment (start 22.22 16.394) (end 21.97 16.144) (width 0.1524) (layer "F.Cu") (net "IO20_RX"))
 (segment (start 10.2348 18.9032) (end 10.2348 19.202622) (width 0.1524) (layer "F.Cu") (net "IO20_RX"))
 (segment (start 10.2348 19.202622) (end 11.151889 20.119711) (width 0.1524) (layer "F.Cu") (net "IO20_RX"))
 (via (at 19.4296 17.3284) (size 0.6) (drill 0.3) (layers "F.Cu" "B.Cu") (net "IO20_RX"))
 (via (at 22.22 16.394) (size 0.6) (drill 0.3) (layers "F.Cu" "B.Cu") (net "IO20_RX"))
 (via (at 10.2348 18.9032) (size 0.6) (drill 0.3) (layers "F.Cu" "B.Cu") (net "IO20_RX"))
 (segment (start 19.764 16.994) (end 19.4296 17.3284) (width 0.1524) (layer "B.Cu") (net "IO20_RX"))
 (segment (start 10.2348 19.0048) (end 10.2348 18.9032) (width 0.1524) (layer "B.Cu") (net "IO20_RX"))
 (segment (start 22.22 16.394) (end 21.62 16.994) (width 0.1524) (layer "B.Cu") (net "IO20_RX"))
 (segment (start 21.62 16.994) (end 19.764 16.994) (width 0.1524) (layer "B.Cu") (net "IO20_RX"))
 (segment (start 20.71 15.36) (end 20.0392 16.0308) (width 0.1524) (layer "F.Cu") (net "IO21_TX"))
 (segment (start 20.91 15.36) (end 20.71 15.36) (width 0.1524) (layer "F.Cu") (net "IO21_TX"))
 (segment (start 20.0392 19.4112) (end 19.5064 19.944) (width 0.1524) (layer "F.Cu") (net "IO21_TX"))
 (segment (start 19.5064 19.944) (end 19.37 19.944) (width 0.1524) (layer "F.Cu") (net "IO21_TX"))
 (segment (start 20.0392 16.0308) (end 20.0392 19.4112) (width 0.1524) (layer "F.Cu") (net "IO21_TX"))
 (segment (start 17.804 19.544011) (end 17.58022 19.767791) (width 0.1524) (layer "F.Cu") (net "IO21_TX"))
 (via (at 19.37 19.944) (size 0.6) (drill 0.3) (layers "F.Cu" "B.Cu") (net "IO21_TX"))
 (via (at 17.804 19.544011) (size 0.6) (drill 0.3) (layers "F.Cu" "B.Cu") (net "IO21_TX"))
 (segment (start 18.546411 19.544011) (end 18.9464 19.944) (width 0.1524) (layer "B.Cu") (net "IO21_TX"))
 (segment (start 17.804 19.544011) (end 18.546411 19.544011) (width 0.1524) (layer "B.Cu") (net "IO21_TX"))
 (segment (start 18.9464 19.944) (end 19.37 19.944) (width 0.1524) (layer "B.Cu") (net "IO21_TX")))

